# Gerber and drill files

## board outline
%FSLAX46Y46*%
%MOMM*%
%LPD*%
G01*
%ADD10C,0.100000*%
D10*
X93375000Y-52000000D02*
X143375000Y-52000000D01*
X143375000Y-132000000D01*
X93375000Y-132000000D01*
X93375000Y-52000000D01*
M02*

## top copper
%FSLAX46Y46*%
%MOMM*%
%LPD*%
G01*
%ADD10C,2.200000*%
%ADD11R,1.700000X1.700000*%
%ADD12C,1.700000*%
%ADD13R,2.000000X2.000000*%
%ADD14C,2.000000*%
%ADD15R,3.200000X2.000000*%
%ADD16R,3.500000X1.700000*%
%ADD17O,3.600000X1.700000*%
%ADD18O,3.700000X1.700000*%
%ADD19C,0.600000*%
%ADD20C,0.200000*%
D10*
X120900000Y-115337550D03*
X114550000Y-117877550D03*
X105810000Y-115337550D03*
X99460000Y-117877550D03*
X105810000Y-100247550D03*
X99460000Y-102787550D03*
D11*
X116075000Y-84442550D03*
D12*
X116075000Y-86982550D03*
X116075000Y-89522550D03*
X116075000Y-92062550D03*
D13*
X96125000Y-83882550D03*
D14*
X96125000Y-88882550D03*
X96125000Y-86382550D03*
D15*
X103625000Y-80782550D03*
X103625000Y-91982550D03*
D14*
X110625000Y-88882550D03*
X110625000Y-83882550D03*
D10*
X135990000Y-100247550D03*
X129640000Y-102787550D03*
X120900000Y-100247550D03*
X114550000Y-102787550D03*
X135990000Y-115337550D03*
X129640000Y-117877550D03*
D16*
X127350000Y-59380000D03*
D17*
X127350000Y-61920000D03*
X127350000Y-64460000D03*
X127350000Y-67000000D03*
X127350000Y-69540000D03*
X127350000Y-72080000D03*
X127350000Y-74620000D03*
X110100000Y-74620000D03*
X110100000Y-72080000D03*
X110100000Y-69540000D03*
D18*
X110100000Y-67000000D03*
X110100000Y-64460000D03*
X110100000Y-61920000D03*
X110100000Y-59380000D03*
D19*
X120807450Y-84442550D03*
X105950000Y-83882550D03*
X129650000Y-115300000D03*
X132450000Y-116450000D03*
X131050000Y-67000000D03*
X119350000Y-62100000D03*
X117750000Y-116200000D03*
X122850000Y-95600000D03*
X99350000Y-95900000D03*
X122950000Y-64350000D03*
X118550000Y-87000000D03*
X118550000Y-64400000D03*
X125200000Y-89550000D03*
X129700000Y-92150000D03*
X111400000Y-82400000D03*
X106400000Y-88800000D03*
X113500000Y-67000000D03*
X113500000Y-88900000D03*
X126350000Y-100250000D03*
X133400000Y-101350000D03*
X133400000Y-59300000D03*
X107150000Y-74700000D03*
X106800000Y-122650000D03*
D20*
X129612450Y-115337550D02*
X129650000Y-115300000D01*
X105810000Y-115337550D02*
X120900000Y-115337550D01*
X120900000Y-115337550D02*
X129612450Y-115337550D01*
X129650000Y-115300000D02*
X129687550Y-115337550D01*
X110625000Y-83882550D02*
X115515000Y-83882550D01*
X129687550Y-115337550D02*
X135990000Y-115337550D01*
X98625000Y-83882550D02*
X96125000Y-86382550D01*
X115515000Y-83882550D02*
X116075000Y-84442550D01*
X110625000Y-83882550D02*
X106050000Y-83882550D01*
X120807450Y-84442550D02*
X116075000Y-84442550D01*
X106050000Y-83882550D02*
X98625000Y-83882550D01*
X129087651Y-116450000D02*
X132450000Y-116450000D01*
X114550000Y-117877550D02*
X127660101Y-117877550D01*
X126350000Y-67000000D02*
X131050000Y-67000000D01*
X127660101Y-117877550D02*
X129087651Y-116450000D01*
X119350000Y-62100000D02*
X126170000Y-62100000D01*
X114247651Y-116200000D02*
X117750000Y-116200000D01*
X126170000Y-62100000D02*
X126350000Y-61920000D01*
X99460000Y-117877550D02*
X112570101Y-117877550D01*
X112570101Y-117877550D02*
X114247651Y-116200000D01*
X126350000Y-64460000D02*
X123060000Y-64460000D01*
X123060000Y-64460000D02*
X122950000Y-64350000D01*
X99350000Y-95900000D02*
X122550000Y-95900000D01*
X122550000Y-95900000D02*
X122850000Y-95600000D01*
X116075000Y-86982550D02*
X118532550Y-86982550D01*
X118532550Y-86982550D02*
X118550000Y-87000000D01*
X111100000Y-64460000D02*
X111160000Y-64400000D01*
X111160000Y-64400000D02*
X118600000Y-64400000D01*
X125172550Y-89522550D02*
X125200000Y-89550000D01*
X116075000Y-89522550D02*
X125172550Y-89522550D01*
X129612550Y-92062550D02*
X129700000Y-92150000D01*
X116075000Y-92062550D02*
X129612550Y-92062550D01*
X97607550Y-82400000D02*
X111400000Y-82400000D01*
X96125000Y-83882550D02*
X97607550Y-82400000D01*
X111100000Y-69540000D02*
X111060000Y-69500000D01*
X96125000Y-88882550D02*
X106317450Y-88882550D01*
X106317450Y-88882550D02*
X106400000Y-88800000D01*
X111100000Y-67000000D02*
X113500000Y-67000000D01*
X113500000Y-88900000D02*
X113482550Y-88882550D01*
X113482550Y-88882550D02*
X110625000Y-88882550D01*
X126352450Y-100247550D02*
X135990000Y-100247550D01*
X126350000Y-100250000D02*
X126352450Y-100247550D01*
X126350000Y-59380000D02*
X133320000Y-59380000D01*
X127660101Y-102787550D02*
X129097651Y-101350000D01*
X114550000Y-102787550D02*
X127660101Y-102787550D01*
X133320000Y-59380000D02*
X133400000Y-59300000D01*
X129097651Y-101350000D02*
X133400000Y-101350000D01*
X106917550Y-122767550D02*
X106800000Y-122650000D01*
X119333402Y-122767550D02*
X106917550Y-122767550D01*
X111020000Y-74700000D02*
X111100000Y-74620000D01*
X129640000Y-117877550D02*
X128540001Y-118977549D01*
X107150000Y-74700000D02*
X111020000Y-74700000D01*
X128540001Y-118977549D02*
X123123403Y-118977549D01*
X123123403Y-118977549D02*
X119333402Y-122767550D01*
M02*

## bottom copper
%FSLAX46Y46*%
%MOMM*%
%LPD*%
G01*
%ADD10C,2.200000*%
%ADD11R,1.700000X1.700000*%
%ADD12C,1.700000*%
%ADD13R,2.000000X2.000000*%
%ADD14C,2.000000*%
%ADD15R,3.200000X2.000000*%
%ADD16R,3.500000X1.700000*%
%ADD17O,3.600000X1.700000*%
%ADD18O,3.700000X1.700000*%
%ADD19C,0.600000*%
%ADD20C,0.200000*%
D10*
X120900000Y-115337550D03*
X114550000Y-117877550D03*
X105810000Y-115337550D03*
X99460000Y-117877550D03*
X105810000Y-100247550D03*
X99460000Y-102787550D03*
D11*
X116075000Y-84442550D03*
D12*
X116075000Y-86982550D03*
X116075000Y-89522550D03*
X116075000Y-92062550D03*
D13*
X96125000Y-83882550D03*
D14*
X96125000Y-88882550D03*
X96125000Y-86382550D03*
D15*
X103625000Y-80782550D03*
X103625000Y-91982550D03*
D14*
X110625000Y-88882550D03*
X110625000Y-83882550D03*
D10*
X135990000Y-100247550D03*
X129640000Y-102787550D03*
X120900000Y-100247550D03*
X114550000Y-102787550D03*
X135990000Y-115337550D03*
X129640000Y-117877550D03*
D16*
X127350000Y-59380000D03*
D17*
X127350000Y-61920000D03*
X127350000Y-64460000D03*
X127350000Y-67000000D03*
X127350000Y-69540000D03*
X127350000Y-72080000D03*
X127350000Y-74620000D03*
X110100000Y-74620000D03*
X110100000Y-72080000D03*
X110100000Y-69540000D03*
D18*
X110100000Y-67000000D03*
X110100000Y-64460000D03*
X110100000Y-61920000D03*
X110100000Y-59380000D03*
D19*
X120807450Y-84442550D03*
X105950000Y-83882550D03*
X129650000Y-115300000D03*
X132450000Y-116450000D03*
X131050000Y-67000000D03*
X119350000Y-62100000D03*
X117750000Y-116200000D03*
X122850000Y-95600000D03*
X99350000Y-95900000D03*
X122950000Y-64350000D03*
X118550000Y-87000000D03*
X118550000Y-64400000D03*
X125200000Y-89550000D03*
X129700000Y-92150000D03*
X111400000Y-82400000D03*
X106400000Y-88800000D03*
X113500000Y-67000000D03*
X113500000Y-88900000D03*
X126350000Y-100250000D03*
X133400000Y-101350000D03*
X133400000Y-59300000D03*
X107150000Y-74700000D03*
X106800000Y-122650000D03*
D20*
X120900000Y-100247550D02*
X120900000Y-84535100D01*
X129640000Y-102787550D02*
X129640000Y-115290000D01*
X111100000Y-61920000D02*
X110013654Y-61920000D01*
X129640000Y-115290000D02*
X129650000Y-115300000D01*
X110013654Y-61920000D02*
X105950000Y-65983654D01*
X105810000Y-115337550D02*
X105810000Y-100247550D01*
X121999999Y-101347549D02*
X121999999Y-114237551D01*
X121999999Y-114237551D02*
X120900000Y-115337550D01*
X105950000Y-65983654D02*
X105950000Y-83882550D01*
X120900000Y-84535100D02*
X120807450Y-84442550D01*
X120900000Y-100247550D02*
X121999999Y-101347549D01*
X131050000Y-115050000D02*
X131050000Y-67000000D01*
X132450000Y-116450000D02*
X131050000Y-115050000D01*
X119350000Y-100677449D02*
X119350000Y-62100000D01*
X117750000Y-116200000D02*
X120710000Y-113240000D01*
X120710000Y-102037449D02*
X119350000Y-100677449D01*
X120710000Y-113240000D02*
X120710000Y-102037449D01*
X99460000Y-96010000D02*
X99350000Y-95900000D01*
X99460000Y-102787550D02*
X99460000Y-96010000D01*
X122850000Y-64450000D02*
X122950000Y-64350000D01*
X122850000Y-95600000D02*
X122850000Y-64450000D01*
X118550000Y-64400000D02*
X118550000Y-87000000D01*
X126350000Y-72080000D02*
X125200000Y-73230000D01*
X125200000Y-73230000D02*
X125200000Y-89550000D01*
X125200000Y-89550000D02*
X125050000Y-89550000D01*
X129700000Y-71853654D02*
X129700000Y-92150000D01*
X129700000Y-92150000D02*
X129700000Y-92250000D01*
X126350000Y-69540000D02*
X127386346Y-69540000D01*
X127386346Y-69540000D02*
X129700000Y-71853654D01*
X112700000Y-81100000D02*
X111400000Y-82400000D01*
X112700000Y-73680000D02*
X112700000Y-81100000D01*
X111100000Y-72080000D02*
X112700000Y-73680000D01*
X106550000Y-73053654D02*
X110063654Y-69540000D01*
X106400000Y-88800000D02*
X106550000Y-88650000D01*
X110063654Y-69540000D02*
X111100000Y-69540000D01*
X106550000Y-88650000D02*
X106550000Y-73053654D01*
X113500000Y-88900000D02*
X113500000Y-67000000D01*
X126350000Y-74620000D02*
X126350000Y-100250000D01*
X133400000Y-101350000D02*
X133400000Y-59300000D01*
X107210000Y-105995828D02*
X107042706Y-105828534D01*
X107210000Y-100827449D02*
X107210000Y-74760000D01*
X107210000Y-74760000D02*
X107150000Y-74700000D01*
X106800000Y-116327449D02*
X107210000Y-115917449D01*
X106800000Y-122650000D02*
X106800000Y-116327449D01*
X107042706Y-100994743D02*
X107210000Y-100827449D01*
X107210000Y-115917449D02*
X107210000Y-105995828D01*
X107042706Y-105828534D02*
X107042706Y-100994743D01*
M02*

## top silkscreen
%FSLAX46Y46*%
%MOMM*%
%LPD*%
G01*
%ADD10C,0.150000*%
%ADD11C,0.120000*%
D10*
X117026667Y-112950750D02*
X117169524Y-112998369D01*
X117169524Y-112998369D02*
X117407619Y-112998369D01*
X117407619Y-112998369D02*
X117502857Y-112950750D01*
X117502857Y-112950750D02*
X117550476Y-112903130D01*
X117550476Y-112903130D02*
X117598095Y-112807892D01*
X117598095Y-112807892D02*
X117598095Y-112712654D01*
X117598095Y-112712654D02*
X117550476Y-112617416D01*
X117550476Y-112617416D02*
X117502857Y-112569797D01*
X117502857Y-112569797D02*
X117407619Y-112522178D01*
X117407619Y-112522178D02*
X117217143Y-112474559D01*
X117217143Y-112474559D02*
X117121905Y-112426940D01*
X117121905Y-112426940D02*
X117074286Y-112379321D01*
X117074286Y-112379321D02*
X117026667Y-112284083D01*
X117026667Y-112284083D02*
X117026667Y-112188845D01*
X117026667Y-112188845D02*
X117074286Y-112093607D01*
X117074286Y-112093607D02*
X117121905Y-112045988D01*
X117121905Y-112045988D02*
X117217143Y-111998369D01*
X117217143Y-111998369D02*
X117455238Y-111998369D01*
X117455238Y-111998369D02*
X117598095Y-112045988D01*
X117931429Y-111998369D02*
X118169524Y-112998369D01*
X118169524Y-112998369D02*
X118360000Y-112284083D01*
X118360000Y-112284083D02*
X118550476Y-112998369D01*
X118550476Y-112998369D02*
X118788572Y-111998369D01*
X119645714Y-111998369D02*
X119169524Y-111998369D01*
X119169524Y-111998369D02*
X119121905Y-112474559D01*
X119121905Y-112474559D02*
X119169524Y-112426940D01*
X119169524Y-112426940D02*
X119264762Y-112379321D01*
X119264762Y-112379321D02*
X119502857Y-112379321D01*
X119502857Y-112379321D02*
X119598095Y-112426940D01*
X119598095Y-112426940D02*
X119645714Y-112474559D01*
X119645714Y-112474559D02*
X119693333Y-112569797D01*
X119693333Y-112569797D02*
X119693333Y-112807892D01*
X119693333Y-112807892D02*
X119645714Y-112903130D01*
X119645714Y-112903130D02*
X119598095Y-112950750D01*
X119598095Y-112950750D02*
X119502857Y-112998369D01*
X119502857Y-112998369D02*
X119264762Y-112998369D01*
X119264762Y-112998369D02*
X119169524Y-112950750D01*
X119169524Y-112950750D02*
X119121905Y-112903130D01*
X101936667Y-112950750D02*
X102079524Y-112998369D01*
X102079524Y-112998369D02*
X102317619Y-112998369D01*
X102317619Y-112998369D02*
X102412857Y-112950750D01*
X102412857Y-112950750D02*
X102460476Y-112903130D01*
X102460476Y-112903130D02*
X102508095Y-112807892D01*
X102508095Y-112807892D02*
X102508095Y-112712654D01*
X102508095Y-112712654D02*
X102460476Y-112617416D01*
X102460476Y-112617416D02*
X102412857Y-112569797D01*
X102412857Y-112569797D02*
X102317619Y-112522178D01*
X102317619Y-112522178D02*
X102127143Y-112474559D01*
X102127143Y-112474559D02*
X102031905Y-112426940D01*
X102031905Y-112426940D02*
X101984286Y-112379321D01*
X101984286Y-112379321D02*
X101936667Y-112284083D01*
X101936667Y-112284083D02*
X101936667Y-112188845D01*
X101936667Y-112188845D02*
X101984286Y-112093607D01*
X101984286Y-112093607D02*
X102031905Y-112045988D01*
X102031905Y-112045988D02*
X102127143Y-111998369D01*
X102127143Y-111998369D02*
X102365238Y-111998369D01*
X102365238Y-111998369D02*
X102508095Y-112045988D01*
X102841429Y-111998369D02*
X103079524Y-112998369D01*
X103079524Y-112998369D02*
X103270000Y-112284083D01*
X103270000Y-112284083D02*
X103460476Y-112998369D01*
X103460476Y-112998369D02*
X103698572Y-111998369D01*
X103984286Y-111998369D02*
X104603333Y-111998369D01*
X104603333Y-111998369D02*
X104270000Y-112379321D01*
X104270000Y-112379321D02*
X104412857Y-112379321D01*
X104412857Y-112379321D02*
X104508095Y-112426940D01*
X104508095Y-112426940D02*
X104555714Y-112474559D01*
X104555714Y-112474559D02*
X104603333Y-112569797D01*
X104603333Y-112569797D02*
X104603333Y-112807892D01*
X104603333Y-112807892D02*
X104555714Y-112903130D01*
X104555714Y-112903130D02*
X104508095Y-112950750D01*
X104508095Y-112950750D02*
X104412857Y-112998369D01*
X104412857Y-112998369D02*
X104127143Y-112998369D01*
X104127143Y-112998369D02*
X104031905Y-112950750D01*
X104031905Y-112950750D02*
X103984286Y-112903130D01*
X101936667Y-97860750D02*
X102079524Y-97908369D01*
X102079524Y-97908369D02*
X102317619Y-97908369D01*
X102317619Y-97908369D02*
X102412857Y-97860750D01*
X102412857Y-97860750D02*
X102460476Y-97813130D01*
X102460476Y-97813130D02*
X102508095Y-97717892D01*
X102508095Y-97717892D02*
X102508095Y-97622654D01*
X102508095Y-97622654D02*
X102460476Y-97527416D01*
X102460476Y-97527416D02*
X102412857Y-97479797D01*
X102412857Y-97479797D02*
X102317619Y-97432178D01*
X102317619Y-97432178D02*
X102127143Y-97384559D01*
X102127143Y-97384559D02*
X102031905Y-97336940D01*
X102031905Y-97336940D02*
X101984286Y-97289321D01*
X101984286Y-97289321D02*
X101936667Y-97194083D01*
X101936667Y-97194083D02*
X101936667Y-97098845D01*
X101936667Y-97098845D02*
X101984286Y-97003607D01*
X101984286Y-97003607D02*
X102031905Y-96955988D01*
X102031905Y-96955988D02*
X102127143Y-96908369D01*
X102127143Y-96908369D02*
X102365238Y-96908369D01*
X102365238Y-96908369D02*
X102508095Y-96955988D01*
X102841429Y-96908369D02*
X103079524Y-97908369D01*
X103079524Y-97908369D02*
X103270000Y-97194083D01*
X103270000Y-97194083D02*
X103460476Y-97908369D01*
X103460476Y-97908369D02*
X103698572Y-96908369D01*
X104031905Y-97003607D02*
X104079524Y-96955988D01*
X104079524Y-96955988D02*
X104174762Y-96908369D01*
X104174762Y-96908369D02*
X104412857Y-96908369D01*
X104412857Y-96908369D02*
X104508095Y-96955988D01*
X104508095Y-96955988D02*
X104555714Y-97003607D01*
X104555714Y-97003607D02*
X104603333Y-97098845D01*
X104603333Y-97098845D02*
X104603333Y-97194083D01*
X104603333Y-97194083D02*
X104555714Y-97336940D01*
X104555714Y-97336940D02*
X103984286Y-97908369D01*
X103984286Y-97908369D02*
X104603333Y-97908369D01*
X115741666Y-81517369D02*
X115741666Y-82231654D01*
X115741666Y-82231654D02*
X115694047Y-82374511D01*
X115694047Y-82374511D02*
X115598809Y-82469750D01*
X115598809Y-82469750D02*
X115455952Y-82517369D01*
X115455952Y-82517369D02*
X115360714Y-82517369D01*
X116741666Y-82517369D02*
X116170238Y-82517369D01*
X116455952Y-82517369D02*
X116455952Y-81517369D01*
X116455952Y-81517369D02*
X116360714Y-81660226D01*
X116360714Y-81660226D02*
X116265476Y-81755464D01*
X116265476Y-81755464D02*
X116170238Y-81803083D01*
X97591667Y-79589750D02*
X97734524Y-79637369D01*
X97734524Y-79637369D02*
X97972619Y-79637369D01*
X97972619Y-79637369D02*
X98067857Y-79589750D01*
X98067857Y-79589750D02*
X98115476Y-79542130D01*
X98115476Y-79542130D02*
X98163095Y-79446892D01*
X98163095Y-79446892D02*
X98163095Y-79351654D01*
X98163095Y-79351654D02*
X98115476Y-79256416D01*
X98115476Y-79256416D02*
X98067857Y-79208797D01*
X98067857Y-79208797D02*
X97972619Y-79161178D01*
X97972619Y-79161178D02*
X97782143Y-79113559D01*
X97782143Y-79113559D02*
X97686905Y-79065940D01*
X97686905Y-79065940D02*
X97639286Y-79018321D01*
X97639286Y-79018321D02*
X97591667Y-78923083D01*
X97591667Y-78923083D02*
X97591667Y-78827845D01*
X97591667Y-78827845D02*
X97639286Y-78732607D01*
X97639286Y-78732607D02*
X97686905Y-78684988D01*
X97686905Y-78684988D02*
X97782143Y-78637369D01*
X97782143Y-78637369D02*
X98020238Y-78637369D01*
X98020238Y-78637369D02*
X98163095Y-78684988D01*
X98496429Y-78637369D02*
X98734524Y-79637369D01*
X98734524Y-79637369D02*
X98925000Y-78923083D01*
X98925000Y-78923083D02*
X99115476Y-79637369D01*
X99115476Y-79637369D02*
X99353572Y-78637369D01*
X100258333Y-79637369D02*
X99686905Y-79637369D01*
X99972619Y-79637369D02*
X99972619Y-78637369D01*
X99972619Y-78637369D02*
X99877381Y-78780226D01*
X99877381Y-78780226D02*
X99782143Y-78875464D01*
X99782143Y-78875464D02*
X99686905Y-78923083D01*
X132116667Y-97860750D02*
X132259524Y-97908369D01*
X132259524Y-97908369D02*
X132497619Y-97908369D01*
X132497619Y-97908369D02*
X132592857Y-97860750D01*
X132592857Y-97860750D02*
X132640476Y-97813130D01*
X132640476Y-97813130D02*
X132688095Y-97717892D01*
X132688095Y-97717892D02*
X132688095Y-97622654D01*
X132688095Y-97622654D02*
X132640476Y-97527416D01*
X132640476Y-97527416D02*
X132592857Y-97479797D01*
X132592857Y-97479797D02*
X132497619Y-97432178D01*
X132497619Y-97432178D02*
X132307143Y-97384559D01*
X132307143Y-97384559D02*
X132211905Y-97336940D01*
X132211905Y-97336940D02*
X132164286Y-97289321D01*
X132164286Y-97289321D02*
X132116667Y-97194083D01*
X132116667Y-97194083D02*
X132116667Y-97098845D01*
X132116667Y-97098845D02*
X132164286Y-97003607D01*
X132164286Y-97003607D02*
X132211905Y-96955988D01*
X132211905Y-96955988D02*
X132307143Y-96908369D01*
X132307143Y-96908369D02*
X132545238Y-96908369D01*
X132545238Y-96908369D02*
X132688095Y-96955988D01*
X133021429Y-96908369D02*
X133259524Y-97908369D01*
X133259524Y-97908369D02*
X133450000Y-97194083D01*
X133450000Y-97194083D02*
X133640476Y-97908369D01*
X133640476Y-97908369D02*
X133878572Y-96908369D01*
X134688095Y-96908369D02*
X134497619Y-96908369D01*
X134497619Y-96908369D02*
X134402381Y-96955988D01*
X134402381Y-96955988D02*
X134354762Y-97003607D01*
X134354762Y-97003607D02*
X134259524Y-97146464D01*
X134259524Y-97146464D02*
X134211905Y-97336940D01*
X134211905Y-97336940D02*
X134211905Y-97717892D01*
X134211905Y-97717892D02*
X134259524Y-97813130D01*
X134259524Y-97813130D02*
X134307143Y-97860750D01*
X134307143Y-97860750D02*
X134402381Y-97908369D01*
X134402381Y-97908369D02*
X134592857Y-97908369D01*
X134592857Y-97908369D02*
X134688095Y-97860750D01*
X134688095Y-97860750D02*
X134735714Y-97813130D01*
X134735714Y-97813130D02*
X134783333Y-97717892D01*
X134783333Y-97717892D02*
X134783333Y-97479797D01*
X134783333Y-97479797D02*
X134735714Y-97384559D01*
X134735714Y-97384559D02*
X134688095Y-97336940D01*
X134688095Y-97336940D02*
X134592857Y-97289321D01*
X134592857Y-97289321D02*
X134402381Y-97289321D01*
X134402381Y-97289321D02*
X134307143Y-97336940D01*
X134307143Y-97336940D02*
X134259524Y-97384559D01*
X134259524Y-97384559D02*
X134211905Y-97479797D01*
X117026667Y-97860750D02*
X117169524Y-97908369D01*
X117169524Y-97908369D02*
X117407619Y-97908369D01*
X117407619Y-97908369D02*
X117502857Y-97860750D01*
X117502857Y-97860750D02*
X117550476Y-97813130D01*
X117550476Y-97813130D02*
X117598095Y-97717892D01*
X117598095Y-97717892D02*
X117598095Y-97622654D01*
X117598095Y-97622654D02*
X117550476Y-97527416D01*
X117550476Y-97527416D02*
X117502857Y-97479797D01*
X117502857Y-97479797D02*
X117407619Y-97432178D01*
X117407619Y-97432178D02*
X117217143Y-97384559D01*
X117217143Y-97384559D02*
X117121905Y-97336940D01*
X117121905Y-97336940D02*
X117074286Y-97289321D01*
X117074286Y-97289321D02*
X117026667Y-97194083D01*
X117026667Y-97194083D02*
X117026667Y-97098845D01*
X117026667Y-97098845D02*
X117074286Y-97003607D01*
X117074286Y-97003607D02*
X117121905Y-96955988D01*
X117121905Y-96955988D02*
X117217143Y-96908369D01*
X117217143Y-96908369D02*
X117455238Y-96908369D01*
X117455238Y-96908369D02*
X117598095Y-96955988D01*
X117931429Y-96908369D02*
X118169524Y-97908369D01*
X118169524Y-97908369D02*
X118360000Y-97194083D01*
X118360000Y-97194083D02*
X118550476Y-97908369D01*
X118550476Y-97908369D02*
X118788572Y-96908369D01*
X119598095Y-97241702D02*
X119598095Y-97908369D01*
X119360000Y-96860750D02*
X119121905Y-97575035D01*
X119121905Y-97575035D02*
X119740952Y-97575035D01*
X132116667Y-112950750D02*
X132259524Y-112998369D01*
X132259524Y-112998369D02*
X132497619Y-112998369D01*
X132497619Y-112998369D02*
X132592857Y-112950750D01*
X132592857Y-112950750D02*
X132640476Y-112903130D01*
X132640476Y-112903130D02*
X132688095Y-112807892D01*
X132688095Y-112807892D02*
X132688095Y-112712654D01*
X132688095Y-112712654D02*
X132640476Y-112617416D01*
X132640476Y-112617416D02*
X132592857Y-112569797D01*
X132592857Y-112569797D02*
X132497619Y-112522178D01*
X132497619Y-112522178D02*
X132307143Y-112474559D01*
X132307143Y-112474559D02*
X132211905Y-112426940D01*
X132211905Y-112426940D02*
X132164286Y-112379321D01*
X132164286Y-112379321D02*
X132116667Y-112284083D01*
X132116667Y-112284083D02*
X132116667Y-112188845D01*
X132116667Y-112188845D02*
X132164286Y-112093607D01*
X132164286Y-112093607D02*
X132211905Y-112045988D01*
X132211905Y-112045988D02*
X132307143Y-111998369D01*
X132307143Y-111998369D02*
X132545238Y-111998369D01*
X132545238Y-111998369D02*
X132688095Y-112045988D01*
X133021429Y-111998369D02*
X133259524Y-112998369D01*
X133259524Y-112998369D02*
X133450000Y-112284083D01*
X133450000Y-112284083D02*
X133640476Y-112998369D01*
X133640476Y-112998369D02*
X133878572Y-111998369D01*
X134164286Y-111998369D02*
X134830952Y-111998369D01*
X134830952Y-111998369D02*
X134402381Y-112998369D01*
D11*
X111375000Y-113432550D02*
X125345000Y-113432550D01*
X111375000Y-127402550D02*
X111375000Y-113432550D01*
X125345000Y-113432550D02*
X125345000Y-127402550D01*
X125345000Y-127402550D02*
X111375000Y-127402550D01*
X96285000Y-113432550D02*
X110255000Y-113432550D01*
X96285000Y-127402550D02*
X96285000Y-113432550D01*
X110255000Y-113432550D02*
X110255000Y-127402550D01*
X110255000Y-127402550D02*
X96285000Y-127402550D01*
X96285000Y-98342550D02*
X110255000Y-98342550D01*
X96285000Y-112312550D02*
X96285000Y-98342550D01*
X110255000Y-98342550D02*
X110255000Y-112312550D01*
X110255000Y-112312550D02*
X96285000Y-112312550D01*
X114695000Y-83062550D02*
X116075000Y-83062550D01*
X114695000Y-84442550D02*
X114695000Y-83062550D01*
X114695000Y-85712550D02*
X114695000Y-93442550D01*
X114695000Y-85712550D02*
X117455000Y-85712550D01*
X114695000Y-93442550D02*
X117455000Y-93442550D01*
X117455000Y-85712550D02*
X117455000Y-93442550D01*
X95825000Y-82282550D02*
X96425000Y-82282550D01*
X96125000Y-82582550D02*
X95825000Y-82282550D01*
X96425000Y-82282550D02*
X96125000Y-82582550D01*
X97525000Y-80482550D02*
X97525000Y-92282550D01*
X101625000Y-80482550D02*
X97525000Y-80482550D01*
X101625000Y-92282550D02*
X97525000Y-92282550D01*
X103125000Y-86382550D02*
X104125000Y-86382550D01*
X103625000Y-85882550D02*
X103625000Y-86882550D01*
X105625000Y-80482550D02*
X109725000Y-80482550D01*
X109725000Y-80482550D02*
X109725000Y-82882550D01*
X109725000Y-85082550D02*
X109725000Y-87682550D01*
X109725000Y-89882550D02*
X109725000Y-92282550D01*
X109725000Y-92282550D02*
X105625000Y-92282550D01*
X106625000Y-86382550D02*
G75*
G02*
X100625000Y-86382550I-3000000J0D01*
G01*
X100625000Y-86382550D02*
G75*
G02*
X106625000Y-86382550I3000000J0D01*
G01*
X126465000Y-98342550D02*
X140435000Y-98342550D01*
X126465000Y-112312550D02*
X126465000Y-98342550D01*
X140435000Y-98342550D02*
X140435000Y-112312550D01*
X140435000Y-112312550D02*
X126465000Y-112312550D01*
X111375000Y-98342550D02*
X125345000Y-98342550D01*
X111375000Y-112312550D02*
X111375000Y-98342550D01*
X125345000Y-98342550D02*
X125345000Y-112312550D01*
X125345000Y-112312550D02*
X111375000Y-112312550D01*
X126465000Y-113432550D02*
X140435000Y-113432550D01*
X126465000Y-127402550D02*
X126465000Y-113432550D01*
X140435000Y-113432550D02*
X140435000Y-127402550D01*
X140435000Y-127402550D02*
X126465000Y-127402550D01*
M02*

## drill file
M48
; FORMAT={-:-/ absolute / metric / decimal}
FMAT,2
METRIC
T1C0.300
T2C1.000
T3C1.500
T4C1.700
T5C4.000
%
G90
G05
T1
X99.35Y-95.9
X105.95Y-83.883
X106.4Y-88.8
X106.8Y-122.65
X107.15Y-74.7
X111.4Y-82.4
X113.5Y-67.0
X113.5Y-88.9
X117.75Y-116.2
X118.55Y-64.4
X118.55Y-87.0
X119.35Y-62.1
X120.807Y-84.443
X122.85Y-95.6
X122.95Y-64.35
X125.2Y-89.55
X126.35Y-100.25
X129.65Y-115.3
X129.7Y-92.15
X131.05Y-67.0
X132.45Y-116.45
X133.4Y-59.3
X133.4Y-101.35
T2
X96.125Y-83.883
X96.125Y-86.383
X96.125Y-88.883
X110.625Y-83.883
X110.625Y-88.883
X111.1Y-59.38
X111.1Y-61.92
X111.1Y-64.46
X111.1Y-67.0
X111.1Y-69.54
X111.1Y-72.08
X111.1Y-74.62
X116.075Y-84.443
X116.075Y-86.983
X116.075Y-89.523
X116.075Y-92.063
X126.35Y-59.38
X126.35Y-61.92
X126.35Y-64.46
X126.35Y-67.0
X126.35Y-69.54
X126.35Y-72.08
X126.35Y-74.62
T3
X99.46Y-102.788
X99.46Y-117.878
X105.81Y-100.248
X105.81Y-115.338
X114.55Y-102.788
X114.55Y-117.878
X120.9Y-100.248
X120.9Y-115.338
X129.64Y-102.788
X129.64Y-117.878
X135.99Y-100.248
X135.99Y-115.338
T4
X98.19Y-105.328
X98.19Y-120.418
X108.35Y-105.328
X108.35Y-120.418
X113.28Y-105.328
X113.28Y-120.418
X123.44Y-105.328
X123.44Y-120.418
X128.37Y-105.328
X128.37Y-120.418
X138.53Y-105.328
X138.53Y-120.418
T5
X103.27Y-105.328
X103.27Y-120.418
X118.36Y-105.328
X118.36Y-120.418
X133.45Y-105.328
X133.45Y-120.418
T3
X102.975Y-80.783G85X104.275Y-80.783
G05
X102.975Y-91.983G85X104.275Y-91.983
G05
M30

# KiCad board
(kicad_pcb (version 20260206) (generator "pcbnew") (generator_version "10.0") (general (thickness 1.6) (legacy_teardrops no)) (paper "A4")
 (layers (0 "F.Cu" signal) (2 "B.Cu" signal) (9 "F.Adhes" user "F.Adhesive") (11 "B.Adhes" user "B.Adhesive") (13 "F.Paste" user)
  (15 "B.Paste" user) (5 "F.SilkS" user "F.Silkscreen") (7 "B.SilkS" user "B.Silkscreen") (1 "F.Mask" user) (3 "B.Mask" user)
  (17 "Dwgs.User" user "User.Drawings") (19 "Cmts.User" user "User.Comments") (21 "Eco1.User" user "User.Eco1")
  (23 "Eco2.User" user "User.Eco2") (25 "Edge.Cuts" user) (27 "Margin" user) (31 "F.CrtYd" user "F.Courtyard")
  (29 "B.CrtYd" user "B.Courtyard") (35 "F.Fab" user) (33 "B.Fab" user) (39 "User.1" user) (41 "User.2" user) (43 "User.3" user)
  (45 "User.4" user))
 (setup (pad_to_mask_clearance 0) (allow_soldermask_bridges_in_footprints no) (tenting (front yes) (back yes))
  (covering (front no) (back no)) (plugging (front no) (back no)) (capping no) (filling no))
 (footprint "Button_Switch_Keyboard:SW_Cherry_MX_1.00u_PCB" (layer "F.Cu") (at 120.9 115.33755)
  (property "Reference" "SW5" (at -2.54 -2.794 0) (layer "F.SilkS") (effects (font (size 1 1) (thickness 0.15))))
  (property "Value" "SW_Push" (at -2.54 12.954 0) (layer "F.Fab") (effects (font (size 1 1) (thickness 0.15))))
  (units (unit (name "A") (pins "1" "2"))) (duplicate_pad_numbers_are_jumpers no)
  (fp_line (start -9.525 -1.905) (end 4.445 -1.905) (stroke (width 0.12) (type solid)) (layer "F.SilkS"))
  (fp_line (start -9.525 12.065) (end -9.525 -1.905) (stroke (width 0.12) (type solid)) (layer "F.SilkS"))
  (fp_line (start 4.445 -1.905) (end 4.445 12.065) (stroke (width 0.12) (type solid)) (layer "F.SilkS"))
  (fp_line (start 4.445 12.065) (end -9.525 12.065) (stroke (width 0.12) (type solid)) (layer "F.SilkS"))
  (pad "" np_thru_hole circle (at -7.62 5.08) (size 1.7 1.7) (drill 1.7) (layers "*.Cu" "*.Mask"))
  (pad "" np_thru_hole circle (at -2.54 5.08) (size 4 4) (drill 4) (layers "*.Cu" "*.Mask"))
  (pad "" np_thru_hole circle (at 2.54 5.08) (size 1.7 1.7) (drill 1.7) (layers "*.Cu" "*.Mask"))
  (pad "1" thru_hole circle (at 0 0) (size 2.2 2.2) (drill 1.5) (layers "*.Cu" "*.Mask") (remove_unused_layers no) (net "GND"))
  (pad "2" thru_hole circle (at -6.35 2.54) (size 2.2 2.2) (drill 1.5) (layers "*.Cu" "*.Mask") (remove_unused_layers no)
   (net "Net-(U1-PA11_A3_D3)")))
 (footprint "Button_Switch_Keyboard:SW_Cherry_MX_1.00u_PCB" (layer "F.Cu") (at 105.81 115.33755)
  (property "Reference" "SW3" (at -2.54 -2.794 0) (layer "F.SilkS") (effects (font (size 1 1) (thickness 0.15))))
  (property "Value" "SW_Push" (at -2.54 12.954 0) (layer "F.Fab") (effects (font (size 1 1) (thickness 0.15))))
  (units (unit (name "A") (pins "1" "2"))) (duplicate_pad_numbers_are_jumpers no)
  (fp_line (start -9.525 -1.905) (end 4.445 -1.905) (stroke (width 0.12) (type solid)) (layer "F.SilkS"))
  (fp_line (start -9.525 12.065) (end -9.525 -1.905) (stroke (width 0.12) (type solid)) (layer "F.SilkS"))
  (fp_line (start 4.445 -1.905) (end 4.445 12.065) (stroke (width 0.12) (type solid)) (layer "F.SilkS"))
  (fp_line (start 4.445 12.065) (end -9.525 12.065) (stroke (width 0.12) (type solid)) (layer "F.SilkS"))
  (pad "" np_thru_hole circle (at -7.62 5.08) (size 1.7 1.7) (drill 1.7) (layers "*.Cu" "*.Mask"))
  (pad "" np_thru_hole circle (at -2.54 5.08) (size 4 4) (drill 4) (layers "*.Cu" "*.Mask"))
  (pad "" np_thru_hole circle (at 2.54 5.08) (size 1.7 1.7) (drill 1.7) (layers "*.Cu" "*.Mask"))
  (pad "1" thru_hole circle (at 0 0) (size 2.2 2.2) (drill 1.5) (layers "*.Cu" "*.Mask") (remove_unused_layers no) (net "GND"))
  (pad "2" thru_hole circle (at -6.35 2.54) (size 2.2 2.2) (drill 1.5) (layers "*.Cu" "*.Mask") (remove_unused_layers no)
   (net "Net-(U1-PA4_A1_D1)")))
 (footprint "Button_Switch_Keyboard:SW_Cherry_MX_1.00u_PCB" (layer "F.Cu") (at 105.81 100.24755)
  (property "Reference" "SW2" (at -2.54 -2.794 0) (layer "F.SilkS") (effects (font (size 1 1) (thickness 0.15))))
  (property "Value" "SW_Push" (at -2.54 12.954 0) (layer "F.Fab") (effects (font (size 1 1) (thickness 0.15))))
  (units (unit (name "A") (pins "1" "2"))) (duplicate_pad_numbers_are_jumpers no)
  (fp_line (start -9.525 -1.905) (end 4.445 -1.905) (stroke (width 0.12) (type solid)) (layer "F.SilkS"))
  (fp_line (start -9.525 12.065) (end -9.525 -1.905) (stroke (width 0.12) (type solid)) (layer "F.SilkS"))
  (fp_line (start 4.445 -1.905) (end 4.445 12.065) (stroke (width 0.12) (type solid)) (layer "F.SilkS"))
  (fp_line (start 4.445 12.065) (end -9.525 12.065) (stroke (width 0.12) (type solid)) (layer "F.SilkS"))
  (pad "" np_thru_hole circle (at -7.62 5.08) (size 1.7 1.7) (drill 1.7) (layers "*.Cu" "*.Mask"))
  (pad "" np_thru_hole circle (at -2.54 5.08) (size 4 4) (drill 4) (layers "*.Cu" "*.Mask"))
  (pad "" np_thru_hole circle (at 2.54 5.08) (size 1.7 1.7) (drill 1.7) (layers "*.Cu" "*.Mask"))
  (pad "1" thru_hole circle (at 0 0) (size 2.2 2.2) (drill 1.5) (layers "*.Cu" "*.Mask") (remove_unused_layers no) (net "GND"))
  (pad "2" thru_hole circle (at -6.35 2.54) (size 2.2 2.2) (drill 1.5) (layers "*.Cu" "*.Mask") (remove_unused_layers no)
   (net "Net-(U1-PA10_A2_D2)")))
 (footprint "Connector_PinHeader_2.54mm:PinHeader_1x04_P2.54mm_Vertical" (layer "F.Cu") (at 116.075 84.44255)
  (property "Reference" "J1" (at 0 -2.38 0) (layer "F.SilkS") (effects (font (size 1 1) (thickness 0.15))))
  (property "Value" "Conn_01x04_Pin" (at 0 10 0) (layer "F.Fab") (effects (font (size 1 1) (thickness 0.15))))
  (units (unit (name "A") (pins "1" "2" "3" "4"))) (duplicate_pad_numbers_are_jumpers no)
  (fp_line (start -1.38 -1.38) (end 0 -1.38) (stroke (width 0.12) (type solid)) (layer "F.SilkS"))
  (fp_line (start -1.38 0) (end -1.38 -1.38) (stroke (width 0.12) (type solid)) (layer "F.SilkS"))
  (fp_line (start -1.38 1.27) (end -1.38 9) (stroke (width 0.12) (type solid)) (layer "F.SilkS"))
  (fp_line (start -1.38 1.27) (end 1.38 1.27) (stroke (width 0.12) (type solid)) (layer "F.SilkS"))
  (fp_line (start -1.38 9) (end 1.38 9) (stroke (width 0.12) (type solid)) (layer "F.SilkS"))
  (fp_line (start 1.38 1.27) (end 1.38 9) (stroke (width 0.12) (type solid)) (layer "F.SilkS"))
  (pad "1" thru_hole rect (at 0 0) (size 1.7 1.7) (drill 1) (layers "*.Cu" "*.Mask") (remove_unused_layers no) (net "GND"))
  (pad "2" thru_hole circle (at 0 2.54) (size 1.7 1.7) (drill 1) (layers "*.Cu" "*.Mask") (remove_unused_layers no) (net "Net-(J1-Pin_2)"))
  (pad "3" thru_hole circle (at 0 5.08) (size 1.7 1.7) (drill 1) (layers "*.Cu" "*.Mask") (remove_unused_layers no) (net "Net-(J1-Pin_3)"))
  (pad "4" thru_hole circle (at 0 7.62) (size 1.7 1.7) (drill 1) (layers "*.Cu" "*.Mask") (remove_unused_layers no) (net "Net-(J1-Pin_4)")))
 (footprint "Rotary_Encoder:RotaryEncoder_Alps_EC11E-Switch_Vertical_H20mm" (layer "F.Cu") (at 96.125 83.88255)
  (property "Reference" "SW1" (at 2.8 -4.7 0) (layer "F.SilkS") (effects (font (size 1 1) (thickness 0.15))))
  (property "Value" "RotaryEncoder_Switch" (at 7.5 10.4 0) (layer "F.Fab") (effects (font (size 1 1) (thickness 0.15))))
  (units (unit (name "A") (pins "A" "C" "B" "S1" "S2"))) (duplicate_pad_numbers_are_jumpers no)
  (fp_line (start -0.3 -1.6) (end 0.3 -1.6) (stroke (width 0.12) (type solid)) (layer "F.SilkS"))
  (fp_line (start 0 -1.3) (end -0.3 -1.6) (stroke (width 0.12) (type solid)) (layer "F.SilkS"))
  (fp_line (start 0.3 -1.6) (end 0 -1.3) (stroke (width 0.12) (type solid)) (layer "F.SilkS"))
  (fp_line (start 1.4 -3.4) (end 1.4 8.4) (stroke (width 0.12) (type solid)) (layer "F.SilkS"))
  (fp_line (start 5.5 -3.4) (end 1.4 -3.4) (stroke (width 0.12) (type solid)) (layer "F.SilkS"))
  (fp_line (start 5.5 8.4) (end 1.4 8.4) (stroke (width 0.12) (type solid)) (layer "F.SilkS"))
  (fp_line (start 7 2.5) (end 8 2.5) (stroke (width 0.12) (type solid)) (layer "F.SilkS"))
  (fp_line (start 7.5 2) (end 7.5 3) (stroke (width 0.12) (type solid)) (layer "F.SilkS"))
  (fp_line (start 9.5 -3.4) (end 13.6 -3.4) (stroke (width 0.12) (type solid)) (layer "F.SilkS"))
  (fp_line (start 13.6 -3.4) (end 13.6 -1) (stroke (width 0.12) (type solid)) (layer "F.SilkS"))
  (fp_line (start 13.6 1.2) (end 13.6 3.8) (stroke (width 0.12) (type solid)) (layer "F.SilkS"))
  (fp_line (start 13.6 6) (end 13.6 8.4) (stroke (width 0.12) (type solid)) (layer "F.SilkS"))
  (fp_line (start 13.6 8.4) (end 9.5 8.4) (stroke (width 0.12) (type solid)) (layer "F.SilkS"))
  (fp_circle (center 7.5 2.5) (end 10.5 2.5) (stroke (width 0.12) (type solid)) (fill no) (layer "F.SilkS"))
  (pad "A" thru_hole rect (at 0 0) (size 2 2) (drill 1) (layers "*.Cu" "*.Mask") (remove_unused_layers no) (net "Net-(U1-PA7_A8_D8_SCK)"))
  (pad "B" thru_hole circle (at 0 5) (size 2 2) (drill 1) (layers "*.Cu" "*.Mask") (remove_unused_layers no) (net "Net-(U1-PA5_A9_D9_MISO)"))
  (pad "C" thru_hole circle (at 0 2.5) (size 2 2) (drill 1) (layers "*.Cu" "*.Mask") (remove_unused_layers no) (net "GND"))
  (pad "MP" thru_hole rect (at 7.5 -3.1) (size 3.2 2) (drill oval 2.8 1.5) (layers "*.Cu" "*.Mask") (remove_unused_layers no))
  (pad "MP" thru_hole rect (at 7.5 8.1) (size 3.2 2) (drill oval 2.8 1.5) (layers "*.Cu" "*.Mask") (remove_unused_layers no))
  (pad "S1" thru_hole circle (at 14.5 5) (size 2 2) (drill 1) (layers "*.Cu" "*.Mask") (remove_unused_layers no)
   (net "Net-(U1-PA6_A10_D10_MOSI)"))
  (pad "S2" thru_hole circle (at 14.5 0) (size 2 2) (drill 1) (layers "*.Cu" "*.Mask") (remove_unused_layers no) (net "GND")))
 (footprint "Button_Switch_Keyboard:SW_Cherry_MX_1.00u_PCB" (layer "F.Cu") (at 135.99 100.24755)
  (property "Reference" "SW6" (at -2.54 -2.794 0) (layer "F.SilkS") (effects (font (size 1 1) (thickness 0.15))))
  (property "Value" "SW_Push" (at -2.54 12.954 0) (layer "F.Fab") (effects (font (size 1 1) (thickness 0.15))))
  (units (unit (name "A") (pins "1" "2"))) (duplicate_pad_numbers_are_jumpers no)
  (fp_line (start -9.525 -1.905) (end 4.445 -1.905) (stroke (width 0.12) (type solid)) (layer "F.SilkS"))
  (fp_line (start -9.525 12.065) (end -9.525 -1.905) (stroke (width 0.12) (type solid)) (layer "F.SilkS"))
  (fp_line (start 4.445 -1.905) (end 4.445 12.065) (stroke (width 0.12) (type solid)) (layer "F.SilkS"))
  (fp_line (start 4.445 12.065) (end -9.525 12.065) (stroke (width 0.12) (type solid)) (layer "F.SilkS"))
  (pad "" np_thru_hole circle (at -7.62 5.08) (size 1.7 1.7) (drill 1.7) (layers "*.Cu" "*.Mask"))
  (pad "" np_thru_hole circle (at -2.54 5.08) (size 4 4) (drill 4) (layers "*.Cu" "*.Mask"))
  (pad "" np_thru_hole circle (at 2.54 5.08) (size 1.7 1.7) (drill 1.7) (layers "*.Cu" "*.Mask"))
  (pad "1" thru_hole circle (at 0 0) (size 2.2 2.2) (drill 1.5) (layers "*.Cu" "*.Mask") (remove_unused_layers no)
   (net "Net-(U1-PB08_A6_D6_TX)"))
  (pad "2" thru_hole circle (at -6.35 2.54) (size 2.2 2.2) (drill 1.5) (layers "*.Cu" "*.Mask") (remove_unused_layers no) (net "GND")))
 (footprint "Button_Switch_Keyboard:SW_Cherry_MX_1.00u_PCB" (layer "F.Cu") (at 120.9 100.24755)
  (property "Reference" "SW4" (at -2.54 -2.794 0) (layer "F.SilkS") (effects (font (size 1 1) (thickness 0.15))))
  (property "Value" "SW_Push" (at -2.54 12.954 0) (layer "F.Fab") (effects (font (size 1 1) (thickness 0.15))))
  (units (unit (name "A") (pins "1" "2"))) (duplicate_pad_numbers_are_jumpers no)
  (fp_line (start -9.525 -1.905) (end 4.445 -1.905) (stroke (width 0.12) (type solid)) (layer "F.SilkS"))
  (fp_line (start -9.525 12.065) (end -9.525 -1.905) (stroke (width 0.12) (type solid)) (layer "F.SilkS"))
  (fp_line (start 4.445 -1.905) (end 4.445 12.065) (stroke (width 0.12) (type solid)) (layer "F.SilkS"))
  (fp_line (start 4.445 12.065) (end -9.525 12.065) (stroke (width 0.12) (type solid)) (layer "F.SilkS"))
  (pad "" np_thru_hole circle (at -7.62 5.08) (size 1.7 1.7) (drill 1.7) (layers "*.Cu" "*.Mask"))
  (pad "" np_thru_hole circle (at -2.54 5.08) (size 4 4) (drill 4) (layers "*.Cu" "*.Mask"))
  (pad "" np_thru_hole circle (at 2.54 5.08) (size 1.7 1.7) (drill 1.7) (layers "*.Cu" "*.Mask"))
  (pad "1" thru_hole circle (at 0 0) (size 2.2 2.2) (drill 1.5) (layers "*.Cu" "*.Mask") (remove_unused_layers no) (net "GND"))
  (pad "2" thru_hole circle (at -6.35 2.54) (size 2.2 2.2) (drill 1.5) (layers "*.Cu" "*.Mask") (remove_unused_layers no)
   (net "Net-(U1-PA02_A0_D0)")))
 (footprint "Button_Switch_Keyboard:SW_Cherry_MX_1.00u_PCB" (layer "F.Cu") (at 135.99 115.33755)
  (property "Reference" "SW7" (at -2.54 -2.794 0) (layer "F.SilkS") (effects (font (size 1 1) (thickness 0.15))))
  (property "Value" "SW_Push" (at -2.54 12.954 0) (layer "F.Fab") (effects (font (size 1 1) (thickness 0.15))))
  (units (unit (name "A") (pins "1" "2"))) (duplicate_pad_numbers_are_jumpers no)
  (fp_line (start -9.525 -1.905) (end 4.445 -1.905) (stroke (width 0.12) (type solid)) (layer "F.SilkS"))
  (fp_line (start -9.525 12.065) (end -9.525 -1.905) (stroke (width 0.12) (type solid)) (layer "F.SilkS"))
  (fp_line (start 4.445 -1.905) (end 4.445 12.065) (stroke (width 0.12) (type solid)) (layer "F.SilkS"))
  (fp_line (start 4.445 12.065) (end -9.525 12.065) (stroke (width 0.12) (type solid)) (layer "F.SilkS"))
  (pad "" np_thru_hole circle (at -7.62 5.08) (size 1.7 1.7) (drill 1.7) (layers "*.Cu" "*.Mask"))
  (pad "" np_thru_hole circle (at -2.54 5.08) (size 4 4) (drill 4) (layers "*.Cu" "*.Mask"))
  (pad "" np_thru_hole circle (at 2.54 5.08) (size 1.7 1.7) (drill 1.7) (layers "*.Cu" "*.Mask"))
  (pad "1" thru_hole circle (at 0 0) (size 2.2 2.2) (drill 1.5) (layers "*.Cu" "*.Mask") (remove_unused_layers no) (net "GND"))
  (pad "2" thru_hole circle (at -6.35 2.54) (size 2.2 2.2) (drill 1.5) (layers "*.Cu" "*.Mask") (remove_unused_layers no)
   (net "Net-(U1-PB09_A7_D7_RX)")))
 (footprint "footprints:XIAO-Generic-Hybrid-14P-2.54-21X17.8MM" (layer "B.Cu") (at 118.725 67 180)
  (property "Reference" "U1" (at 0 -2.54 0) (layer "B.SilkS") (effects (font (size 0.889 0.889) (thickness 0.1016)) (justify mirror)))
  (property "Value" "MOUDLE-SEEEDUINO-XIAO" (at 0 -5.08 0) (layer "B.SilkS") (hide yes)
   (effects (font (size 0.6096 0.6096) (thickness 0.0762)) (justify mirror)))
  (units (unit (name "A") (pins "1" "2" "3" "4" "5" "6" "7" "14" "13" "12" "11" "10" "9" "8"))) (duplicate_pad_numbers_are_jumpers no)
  (pad "1" thru_hole rect (at -7.625 7.62 180) (size 3.5 1.7) (drill 1 (offset -1 0)) (layers "*.Cu" "*.Mask") (remove_unused_layers no)
   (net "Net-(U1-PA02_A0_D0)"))
  (pad "2" thru_hole oval (at -7.625 5.08 180) (size 3.6 1.7) (drill 1 (offset -1 0)) (layers "*.Cu" "*.Mask") (remove_unused_layers no)
   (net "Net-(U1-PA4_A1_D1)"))
  (pad "3" thru_hole oval (at -7.625 2.54 180) (size 3.6 1.7) (drill 1 (offset -1 0)) (layers "*.Cu" "*.Mask") (remove_unused_layers no)
   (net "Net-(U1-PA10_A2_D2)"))
  (pad "4" thru_hole oval (at -7.625 0 180) (size 3.6 1.7) (drill 1 (offset -1 0)) (layers "*.Cu" "*.Mask") (remove_unused_layers no)
   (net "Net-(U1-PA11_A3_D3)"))
  (pad "5" thru_hole oval (at -7.625 -2.54 180) (size 3.6 1.7) (drill 1 (offset -1 0)) (layers "*.Cu" "*.Mask") (remove_unused_layers no)
   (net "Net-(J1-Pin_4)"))
  (pad "6" thru_hole oval (at -7.625 -5.08) (size 3.6 1.7) (drill 1 (offset 1 0)) (layers "*.Cu" "*.Mask") (remove_unused_layers no)
   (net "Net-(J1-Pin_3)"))
  (pad "7" thru_hole oval (at -7.625 -7.62 180) (size 3.6 1.7) (drill 1 (offset -1 0)) (layers "*.Cu" "*.Mask") (remove_unused_layers no)
   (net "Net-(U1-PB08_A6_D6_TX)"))
  (pad "8" thru_hole oval (at 7.625 -7.62 180) (size 3.6 1.7) (drill 1 (offset 1 0)) (layers "*.Cu" "*.Mask") (remove_unused_layers no)
   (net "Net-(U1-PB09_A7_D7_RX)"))
  (pad "9" thru_hole oval (at 7.625 -5.08 180) (size 3.6 1.7) (drill 1 (offset 1 0)) (layers "*.Cu" "*.Mask") (remove_unused_layers no)
   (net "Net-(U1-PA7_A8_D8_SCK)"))
  (pad "10" thru_hole oval (at 7.625 -2.54 180) (size 3.6 1.7) (drill 1 (offset 1 0)) (layers "*.Cu" "*.Mask") (remove_unused_layers no)
   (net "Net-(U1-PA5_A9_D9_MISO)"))
  (pad "11" thru_hole oval (at 7.625 0 180) (size 3.7 1.7) (drill 1 (offset 1 0)) (layers "*.Cu" "*.Mask") (remove_unused_layers no)
   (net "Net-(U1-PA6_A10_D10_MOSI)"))
  (pad "12" thru_hole oval (at 7.625 2.54 180) (size 3.7 1.7) (drill 1 (offset 1 0)) (layers "*.Cu" "*.Mask") (remove_unused_layers no)
   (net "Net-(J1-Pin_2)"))
  (pad "13" thru_hole oval (at 7.625 5.08 180) (size 3.7 1.7) (drill 1 (offset 1 0)) (layers "*.Cu" "*.Mask") (remove_unused_layers no)
   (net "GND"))
  (pad "14" thru_hole oval (at 7.625 7.62 180) (size 3.7 1.7) (drill 1 (offset 1 0)) (layers "*.Cu" "*.Mask") (remove_unused_layers no)
   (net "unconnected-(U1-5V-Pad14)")))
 (gr_rect (start 93.375 52) (end 143.375 132) (stroke (width 0.1) (type solid)) (fill no) (layer "Edge.Cuts"))
 (segment (start 129.61245 115.33755) (end 129.65 115.3) (width 0.2) (layer "F.Cu") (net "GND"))
 (segment (start 105.81 115.33755) (end 120.9 115.33755) (width 0.2) (layer "F.Cu") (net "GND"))
 (segment (start 120.9 115.33755) (end 129.61245 115.33755) (width 0.2) (layer "F.Cu") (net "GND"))
 (segment (start 129.65 115.3) (end 129.68755 115.33755) (width 0.2) (layer "F.Cu") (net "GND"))
 (segment (start 110.625 83.88255) (end 115.515 83.88255) (width 0.2) (layer "F.Cu") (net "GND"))
 (segment (start 129.68755 115.33755) (end 135.99 115.33755) (width 0.2) (layer "F.Cu") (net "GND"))
 (segment (start 98.625 83.88255) (end 96.125 86.38255) (width 0.2) (layer "F.Cu") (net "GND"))
 (segment (start 115.515 83.88255) (end 116.075 84.44255) (width 0.2) (layer "F.Cu") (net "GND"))
 (segment (start 110.625 83.88255) (end 106.05 83.88255) (width 0.2) (layer "F.Cu") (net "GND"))
 (segment (start 120.80745 84.44255) (end 116.075 84.44255) (width 0.2) (layer "F.Cu") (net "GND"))
 (segment (start 106.05 83.88255) (end 98.625 83.88255) (width 0.2) (layer "F.Cu") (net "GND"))
 (via (at 120.80745 84.44255) (size 0.6) (drill 0.3) (layers "F.Cu" "B.Cu") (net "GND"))
 (via (at 105.95 83.88255) (size 0.6) (drill 0.3) (layers "F.Cu" "B.Cu") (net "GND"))
 (via (at 129.65 115.3) (size 0.6) (drill 0.3) (layers "F.Cu" "B.Cu") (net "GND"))
 (segment (start 120.9 100.24755) (end 120.9 84.5351) (width 0.2) (layer "B.Cu") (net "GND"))
 (segment (start 129.64 102.78755) (end 129.64 115.29) (width 0.2) (layer "B.Cu") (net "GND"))
 (segment (start 111.1 61.92) (end 110.013654 61.92) (width 0.2) (layer "B.Cu") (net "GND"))
 (segment (start 129.64 115.29) (end 129.65 115.3) (width 0.2) (layer "B.Cu") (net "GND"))
 (segment (start 110.013654 61.92) (end 105.95 65.983654) (width 0.2) (layer "B.Cu") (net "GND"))
 (segment (start 105.81 115.33755) (end 105.81 100.24755) (width 0.2) (layer "B.Cu") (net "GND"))
 (segment (start 121.999999 101.347549) (end 121.999999 114.237551) (width 0.2) (layer "B.Cu") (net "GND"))
 (segment (start 121.999999 114.237551) (end 120.9 115.33755) (width 0.2) (layer "B.Cu") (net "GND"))
 (segment (start 105.95 65.983654) (end 105.95 83.88255) (width 0.2) (layer "B.Cu") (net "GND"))
 (segment (start 120.9 84.5351) (end 120.80745 84.44255) (width 0.2) (layer "B.Cu") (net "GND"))
 (segment (start 120.9 100.24755) (end 121.999999 101.347549) (width 0.2) (layer "B.Cu") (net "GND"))
 (segment (start 129.087651 116.45) (end 132.45 116.45) (width 0.2) (layer "F.Cu") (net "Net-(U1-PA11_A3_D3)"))
 (segment (start 114.55 117.87755) (end 127.660101 117.87755) (width 0.2) (layer "F.Cu") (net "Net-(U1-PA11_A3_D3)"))
 (segment (start 126.35 67) (end 131.05 67) (width 0.2) (layer "F.Cu") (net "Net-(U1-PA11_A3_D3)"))
 (segment (start 127.660101 117.87755) (end 129.087651 116.45) (width 0.2) (layer "F.Cu") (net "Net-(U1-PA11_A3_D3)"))
 (via (at 132.45 116.45) (size 0.6) (drill 0.3) (layers "F.Cu" "B.Cu") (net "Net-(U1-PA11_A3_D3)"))
 (via (at 131.05 67) (size 0.6) (drill 0.3) (layers "F.Cu" "B.Cu") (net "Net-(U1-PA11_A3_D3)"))
 (segment (start 131.05 115.05) (end 131.05 67) (width 0.2) (layer "B.Cu") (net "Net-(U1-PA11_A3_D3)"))
 (segment (start 132.45 116.45) (end 131.05 115.05) (width 0.2) (layer "B.Cu") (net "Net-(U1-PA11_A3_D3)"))
 (segment (start 119.35 62.1) (end 126.17 62.1) (width 0.2) (layer "F.Cu") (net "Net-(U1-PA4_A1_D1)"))
 (segment (start 114.247651 116.2) (end 117.75 116.2) (width 0.2) (layer "F.Cu") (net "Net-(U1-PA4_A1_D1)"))
 (segment (start 126.17 62.1) (end 126.35 61.92) (width 0.2) (layer "F.Cu") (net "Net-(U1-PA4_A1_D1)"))
 (segment (start 99.46 117.87755) (end 112.570101 117.87755) (width 0.2) (layer "F.Cu") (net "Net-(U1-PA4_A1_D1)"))
 (segment (start 112.570101 117.87755) (end 114.247651 116.2) (width 0.2) (layer "F.Cu") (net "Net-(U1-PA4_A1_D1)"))
 (via (at 119.35 62.1) (size 0.6) (drill 0.3) (layers "F.Cu" "B.Cu") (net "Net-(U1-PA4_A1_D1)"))
 (via (at 117.75 116.2) (size 0.6) (drill 0.3) (layers "F.Cu" "B.Cu") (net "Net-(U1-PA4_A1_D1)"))
 (segment (start 119.35 100.677449) (end 119.35 62.1) (width 0.2) (layer "B.Cu") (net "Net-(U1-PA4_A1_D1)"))
 (segment (start 117.75 116.2) (end 120.71 113.24) (width 0.2) (layer "B.Cu") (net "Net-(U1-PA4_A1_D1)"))
 (segment (start 120.71 102.037449) (end 119.35 100.677449) (width 0.2) (layer "B.Cu") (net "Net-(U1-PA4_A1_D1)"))
 (segment (start 120.71 113.24) (end 120.71 102.037449) (width 0.2) (layer "B.Cu") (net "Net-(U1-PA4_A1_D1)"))
 (segment (start 126.35 64.46) (end 123.06 64.46) (width 0.2) (layer "F.Cu") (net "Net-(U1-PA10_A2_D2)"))
 (segment (start 123.06 64.46) (end 122.95 64.35) (width 0.2) (layer "F.Cu") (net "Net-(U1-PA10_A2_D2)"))
 (segment (start 99.35 95.9) (end 122.55 95.9) (width 0.2) (layer "F.Cu") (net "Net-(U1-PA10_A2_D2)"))
 (segment (start 122.55 95.9) (end 122.85 95.6) (width 0.2) (layer "F.Cu") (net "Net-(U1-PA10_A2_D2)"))
 (via (at 122.85 95.6) (size 0.6) (drill 0.3) (layers "F.Cu" "B.Cu") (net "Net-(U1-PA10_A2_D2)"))
 (via (at 99.35 95.9) (size 0.6) (drill 0.3) (layers "F.Cu" "B.Cu") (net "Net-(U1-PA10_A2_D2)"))
 (via (at 122.95 64.35) (size 0.6) (drill 0.3) (layers "F.Cu" "B.Cu") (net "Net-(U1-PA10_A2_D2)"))
 (segment (start 99.46 96.01) (end 99.35 95.9) (width 0.2) (layer "B.Cu") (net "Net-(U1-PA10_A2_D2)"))
 (segment (start 99.46 102.78755) (end 99.46 96.01) (width 0.2) (layer "B.Cu") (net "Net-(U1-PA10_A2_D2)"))
 (segment (start 122.85 64.45) (end 122.95 64.35) (width 0.2) (layer "B.Cu") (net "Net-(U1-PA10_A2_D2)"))
 (segment (start 122.85 95.6) (end 122.85 64.45) (width 0.2) (layer "B.Cu") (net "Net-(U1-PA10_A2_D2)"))
 (segment (start 116.075 86.98255) (end 118.53255 86.98255) (width 0.2) (layer "F.Cu") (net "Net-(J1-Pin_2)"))
 (segment (start 118.53255 86.98255) (end 118.55 87) (width 0.2) (layer "F.Cu") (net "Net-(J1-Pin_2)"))
 (segment (start 111.1 64.46) (end 111.16 64.4) (width 0.2) (layer "F.Cu") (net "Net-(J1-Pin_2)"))
 (segment (start 111.16 64.4) (end 118.6 64.4) (width 0.2) (layer "F.Cu") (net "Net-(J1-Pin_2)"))
 (via (at 118.55 87) (size 0.6) (drill 0.3) (layers "F.Cu" "B.Cu") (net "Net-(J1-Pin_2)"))
 (via (at 118.55 64.4) (size 0.6) (drill 0.3) (layers "F.Cu" "B.Cu") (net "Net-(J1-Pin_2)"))
 (segment (start 118.55 64.4) (end 118.55 87) (width 0.2) (layer "B.Cu") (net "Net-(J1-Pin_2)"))
 (segment (start 125.17255 89.52255) (end 125.2 89.55) (width 0.2) (layer "F.Cu") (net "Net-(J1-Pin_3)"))
 (segment (start 116.075 89.52255) (end 125.17255 89.52255) (width 0.2) (layer "F.Cu") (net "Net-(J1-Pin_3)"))
 (via (at 125.2 89.55) (size 0.6) (drill 0.3) (layers "F.Cu" "B.Cu") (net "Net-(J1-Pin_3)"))
 (segment (start 126.35 72.08) (end 125.2 73.23) (width 0.2) (layer "B.Cu") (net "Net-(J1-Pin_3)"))
 (segment (start 125.2 73.23) (end 125.2 89.55) (width 0.2) (layer "B.Cu") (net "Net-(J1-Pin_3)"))
 (segment (start 125.2 89.55) (end 125.05 89.55) (width 0.2) (layer "B.Cu") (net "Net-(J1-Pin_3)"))
 (segment (start 129.61255 92.06255) (end 129.7 92.15) (width 0.2) (layer "F.Cu") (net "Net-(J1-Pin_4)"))
 (segment (start 116.075 92.06255) (end 129.61255 92.06255) (width 0.2) (layer "F.Cu") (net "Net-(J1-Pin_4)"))
 (via (at 129.7 92.15) (size 0.6) (drill 0.3) (layers "F.Cu" "B.Cu") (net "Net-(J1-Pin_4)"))
 (segment (start 129.7 71.853654) (end 129.7 92.15) (width 0.2) (layer "B.Cu") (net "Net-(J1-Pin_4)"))
 (segment (start 129.7 92.15) (end 129.7 92.25) (width 0.2) (layer "B.Cu") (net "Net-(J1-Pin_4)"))
 (segment (start 126.35 69.54) (end 127.386346 69.54) (width 0.2) (layer "B.Cu") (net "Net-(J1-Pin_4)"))
 (segment (start 127.386346 69.54) (end 129.7 71.853654) (width 0.2) (layer "B.Cu") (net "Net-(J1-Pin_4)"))
 (segment (start 97.60755 82.4) (end 111.4 82.4) (width 0.2) (layer "F.Cu") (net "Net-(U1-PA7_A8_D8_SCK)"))
 (segment (start 96.125 83.88255) (end 97.60755 82.4) (width 0.2) (layer "F.Cu") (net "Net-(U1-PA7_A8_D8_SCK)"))
 (via (at 111.4 82.4) (size 0.6) (drill 0.3) (layers "F.Cu" "B.Cu") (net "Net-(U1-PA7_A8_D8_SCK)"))
 (segment (start 112.7 81.1) (end 111.4 82.4) (width 0.2) (layer "B.Cu") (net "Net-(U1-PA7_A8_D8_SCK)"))
 (segment (start 112.7 73.68) (end 112.7 81.1) (width 0.2) (layer "B.Cu") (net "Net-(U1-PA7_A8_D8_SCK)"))
 (segment (start 111.1 72.08) (end 112.7 73.68) (width 0.2) (layer "B.Cu") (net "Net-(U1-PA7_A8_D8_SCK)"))
 (segment (start 111.1 69.54) (end 111.06 69.5) (width 0.2) (layer "F.Cu") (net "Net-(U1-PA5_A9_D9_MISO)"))
 (segment (start 96.125 88.88255) (end 106.31745 88.88255) (width 0.2) (layer "F.Cu") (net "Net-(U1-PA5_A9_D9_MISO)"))
 (segment (start 106.31745 88.88255) (end 106.4 88.8) (width 0.2) (layer "F.Cu") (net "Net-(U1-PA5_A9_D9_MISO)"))
 (via (at 106.4 88.8) (size 0.6) (drill 0.3) (layers "F.Cu" "B.Cu") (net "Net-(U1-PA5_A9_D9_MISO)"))
 (segment (start 106.55 73.053654) (end 110.063654 69.54) (width 0.2) (layer "B.Cu") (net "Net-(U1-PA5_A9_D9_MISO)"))
 (segment (start 106.4 88.8) (end 106.55 88.65) (width 0.2) (layer "B.Cu") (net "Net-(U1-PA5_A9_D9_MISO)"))
 (segment (start 110.063654 69.54) (end 111.1 69.54) (width 0.2) (layer "B.Cu") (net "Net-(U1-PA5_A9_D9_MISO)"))
 (segment (start 106.55 88.65) (end 106.55 73.053654) (width 0.2) (layer "B.Cu") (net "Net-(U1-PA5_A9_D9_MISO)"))
 (segment (start 111.1 67) (end 113.5 67) (width 0.2) (layer "F.Cu") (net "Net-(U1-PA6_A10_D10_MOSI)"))
 (segment (start 113.5 88.9) (end 113.48255 88.88255) (width 0.2) (layer "F.Cu") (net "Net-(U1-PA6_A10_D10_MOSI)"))
 (segment (start 113.48255 88.88255) (end 110.625 88.88255) (width 0.2) (layer "F.Cu") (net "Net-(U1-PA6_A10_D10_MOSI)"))
 (via (at 113.5 67) (size 0.6) (drill 0.3) (layers "F.Cu" "B.Cu") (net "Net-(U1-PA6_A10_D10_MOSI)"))
 (via (at 113.5 88.9) (size 0.6) (drill 0.3) (layers "F.Cu" "B.Cu") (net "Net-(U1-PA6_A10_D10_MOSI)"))
 (segment (start 113.5 88.9) (end 113.5 67) (width 0.2) (layer "B.Cu") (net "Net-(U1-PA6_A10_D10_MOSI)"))
 (segment (start 126.35245 100.24755) (end 135.99 100.24755) (width 0.2) (layer "F.Cu") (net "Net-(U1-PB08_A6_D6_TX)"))
 (segment (start 126.35 100.25) (end 126.35245 100.24755) (width 0.2) (layer "F.Cu") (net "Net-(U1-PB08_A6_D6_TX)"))
 (via (at 126.35 100.25) (size 0.6) (drill 0.3) (layers "F.Cu" "B.Cu") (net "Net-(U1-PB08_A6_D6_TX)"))
 (segment (start 126.35 74.62) (end 126.35 100.25) (width 0.2) (layer "B.Cu") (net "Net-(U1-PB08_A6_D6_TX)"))
 (segment (start 126.35 59.38) (end 133.32 59.38) (width 0.2) (layer "F.Cu") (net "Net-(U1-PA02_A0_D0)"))
 (segment (start 127.660101 102.78755) (end 129.097651 101.35) (width 0.2) (layer "F.Cu") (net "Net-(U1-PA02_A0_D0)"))
 (segment (start 114.55 102.78755) (end 127.660101 102.78755) (width 0.2) (layer "F.Cu") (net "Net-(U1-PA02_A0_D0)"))
 (segment (start 133.32 59.38) (end 133.4 59.3) (width 0.2) (layer "F.Cu") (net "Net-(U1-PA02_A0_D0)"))
 (segment (start 129.097651 101.35) (end 133.4 101.35) (width 0.2) (layer "F.Cu") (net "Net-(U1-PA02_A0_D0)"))
 (via (at 133.4 101.35) (size 0.6) (drill 0.3) (layers "F.Cu" "B.Cu") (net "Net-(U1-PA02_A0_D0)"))
 (via (at 133.4 59.3) (size 0.6) (drill 0.3) (layers "F.Cu" "B.Cu") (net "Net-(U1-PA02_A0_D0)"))
 (segment (start 133.4 101.35) (end 133.4 59.3) (width 0.2) (layer "B.Cu") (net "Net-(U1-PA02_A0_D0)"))
 (segment (start 106.91755 122.76755) (end 106.8 122.65) (width 0.2) (layer "F.Cu") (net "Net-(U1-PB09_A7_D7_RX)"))
 (segment (start 119.333402 122.76755) (end 106.91755 122.76755) (width 0.2) (layer "F.Cu") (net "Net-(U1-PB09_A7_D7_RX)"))
 (segment (start 111.02 74.7) (end 111.1 74.62) (width 0.2) (layer "F.Cu") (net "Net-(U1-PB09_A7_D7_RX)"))
 (segment (start 129.64 117.87755) (end 128.540001 118.977549) (width 0.2) (layer "F.Cu") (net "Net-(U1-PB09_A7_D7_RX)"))
 (segment (start 107.15 74.7) (end 111.02 74.7) (width 0.2) (layer "F.Cu") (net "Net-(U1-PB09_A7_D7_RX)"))
 (segment (start 128.540001 118.977549) (end 123.123403 118.977549) (width 0.2) (layer "F.Cu") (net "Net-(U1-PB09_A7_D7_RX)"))
 (segment (start 123.123403 118.977549) (end 119.333402 122.76755) (width 0.2) (layer "F.Cu") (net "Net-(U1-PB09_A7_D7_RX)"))
 (via (at 107.15 74.7) (size 0.6) (drill 0.3) (layers "F.Cu" "B.Cu") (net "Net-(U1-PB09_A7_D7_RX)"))
 (via (at 106.8 122.65) (size 0.6) (drill 0.3) (layers "F.Cu" "B.Cu") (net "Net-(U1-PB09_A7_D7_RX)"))
 (segment (start 107.21 105.995828) (end 107.042706 105.828534) (width 0.2) (layer "B.Cu") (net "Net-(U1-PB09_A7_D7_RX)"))
 (segment (start 107.21 100.827449) (end 107.21 74.76) (width 0.2) (layer "B.Cu") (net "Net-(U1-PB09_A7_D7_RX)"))
 (segment (start 107.21 74.76) (end 107.15 74.7) (width 0.2) (layer "B.Cu") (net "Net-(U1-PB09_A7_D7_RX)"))
 (segment (start 106.8 116.327449) (end 107.21 115.917449) (width 0.2) (layer "B.Cu") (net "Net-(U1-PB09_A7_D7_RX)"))
 (segment (start 106.8 122.65) (end 106.8 116.327449) (width 0.2) (layer "B.Cu") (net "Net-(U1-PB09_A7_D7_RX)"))
 (segment (start 107.042706 100.994743) (end 107.21 100.827449) (width 0.2) (layer "B.Cu") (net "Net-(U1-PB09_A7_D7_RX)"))
 (segment (start 107.21 115.917449) (end 107.21 105.995828) (width 0.2) (layer "B.Cu") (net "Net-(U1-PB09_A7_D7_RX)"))
 (segment (start 107.042706 105.828534) (end 107.042706 100.994743) (width 0.2) (layer "B.Cu") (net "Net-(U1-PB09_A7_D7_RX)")))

